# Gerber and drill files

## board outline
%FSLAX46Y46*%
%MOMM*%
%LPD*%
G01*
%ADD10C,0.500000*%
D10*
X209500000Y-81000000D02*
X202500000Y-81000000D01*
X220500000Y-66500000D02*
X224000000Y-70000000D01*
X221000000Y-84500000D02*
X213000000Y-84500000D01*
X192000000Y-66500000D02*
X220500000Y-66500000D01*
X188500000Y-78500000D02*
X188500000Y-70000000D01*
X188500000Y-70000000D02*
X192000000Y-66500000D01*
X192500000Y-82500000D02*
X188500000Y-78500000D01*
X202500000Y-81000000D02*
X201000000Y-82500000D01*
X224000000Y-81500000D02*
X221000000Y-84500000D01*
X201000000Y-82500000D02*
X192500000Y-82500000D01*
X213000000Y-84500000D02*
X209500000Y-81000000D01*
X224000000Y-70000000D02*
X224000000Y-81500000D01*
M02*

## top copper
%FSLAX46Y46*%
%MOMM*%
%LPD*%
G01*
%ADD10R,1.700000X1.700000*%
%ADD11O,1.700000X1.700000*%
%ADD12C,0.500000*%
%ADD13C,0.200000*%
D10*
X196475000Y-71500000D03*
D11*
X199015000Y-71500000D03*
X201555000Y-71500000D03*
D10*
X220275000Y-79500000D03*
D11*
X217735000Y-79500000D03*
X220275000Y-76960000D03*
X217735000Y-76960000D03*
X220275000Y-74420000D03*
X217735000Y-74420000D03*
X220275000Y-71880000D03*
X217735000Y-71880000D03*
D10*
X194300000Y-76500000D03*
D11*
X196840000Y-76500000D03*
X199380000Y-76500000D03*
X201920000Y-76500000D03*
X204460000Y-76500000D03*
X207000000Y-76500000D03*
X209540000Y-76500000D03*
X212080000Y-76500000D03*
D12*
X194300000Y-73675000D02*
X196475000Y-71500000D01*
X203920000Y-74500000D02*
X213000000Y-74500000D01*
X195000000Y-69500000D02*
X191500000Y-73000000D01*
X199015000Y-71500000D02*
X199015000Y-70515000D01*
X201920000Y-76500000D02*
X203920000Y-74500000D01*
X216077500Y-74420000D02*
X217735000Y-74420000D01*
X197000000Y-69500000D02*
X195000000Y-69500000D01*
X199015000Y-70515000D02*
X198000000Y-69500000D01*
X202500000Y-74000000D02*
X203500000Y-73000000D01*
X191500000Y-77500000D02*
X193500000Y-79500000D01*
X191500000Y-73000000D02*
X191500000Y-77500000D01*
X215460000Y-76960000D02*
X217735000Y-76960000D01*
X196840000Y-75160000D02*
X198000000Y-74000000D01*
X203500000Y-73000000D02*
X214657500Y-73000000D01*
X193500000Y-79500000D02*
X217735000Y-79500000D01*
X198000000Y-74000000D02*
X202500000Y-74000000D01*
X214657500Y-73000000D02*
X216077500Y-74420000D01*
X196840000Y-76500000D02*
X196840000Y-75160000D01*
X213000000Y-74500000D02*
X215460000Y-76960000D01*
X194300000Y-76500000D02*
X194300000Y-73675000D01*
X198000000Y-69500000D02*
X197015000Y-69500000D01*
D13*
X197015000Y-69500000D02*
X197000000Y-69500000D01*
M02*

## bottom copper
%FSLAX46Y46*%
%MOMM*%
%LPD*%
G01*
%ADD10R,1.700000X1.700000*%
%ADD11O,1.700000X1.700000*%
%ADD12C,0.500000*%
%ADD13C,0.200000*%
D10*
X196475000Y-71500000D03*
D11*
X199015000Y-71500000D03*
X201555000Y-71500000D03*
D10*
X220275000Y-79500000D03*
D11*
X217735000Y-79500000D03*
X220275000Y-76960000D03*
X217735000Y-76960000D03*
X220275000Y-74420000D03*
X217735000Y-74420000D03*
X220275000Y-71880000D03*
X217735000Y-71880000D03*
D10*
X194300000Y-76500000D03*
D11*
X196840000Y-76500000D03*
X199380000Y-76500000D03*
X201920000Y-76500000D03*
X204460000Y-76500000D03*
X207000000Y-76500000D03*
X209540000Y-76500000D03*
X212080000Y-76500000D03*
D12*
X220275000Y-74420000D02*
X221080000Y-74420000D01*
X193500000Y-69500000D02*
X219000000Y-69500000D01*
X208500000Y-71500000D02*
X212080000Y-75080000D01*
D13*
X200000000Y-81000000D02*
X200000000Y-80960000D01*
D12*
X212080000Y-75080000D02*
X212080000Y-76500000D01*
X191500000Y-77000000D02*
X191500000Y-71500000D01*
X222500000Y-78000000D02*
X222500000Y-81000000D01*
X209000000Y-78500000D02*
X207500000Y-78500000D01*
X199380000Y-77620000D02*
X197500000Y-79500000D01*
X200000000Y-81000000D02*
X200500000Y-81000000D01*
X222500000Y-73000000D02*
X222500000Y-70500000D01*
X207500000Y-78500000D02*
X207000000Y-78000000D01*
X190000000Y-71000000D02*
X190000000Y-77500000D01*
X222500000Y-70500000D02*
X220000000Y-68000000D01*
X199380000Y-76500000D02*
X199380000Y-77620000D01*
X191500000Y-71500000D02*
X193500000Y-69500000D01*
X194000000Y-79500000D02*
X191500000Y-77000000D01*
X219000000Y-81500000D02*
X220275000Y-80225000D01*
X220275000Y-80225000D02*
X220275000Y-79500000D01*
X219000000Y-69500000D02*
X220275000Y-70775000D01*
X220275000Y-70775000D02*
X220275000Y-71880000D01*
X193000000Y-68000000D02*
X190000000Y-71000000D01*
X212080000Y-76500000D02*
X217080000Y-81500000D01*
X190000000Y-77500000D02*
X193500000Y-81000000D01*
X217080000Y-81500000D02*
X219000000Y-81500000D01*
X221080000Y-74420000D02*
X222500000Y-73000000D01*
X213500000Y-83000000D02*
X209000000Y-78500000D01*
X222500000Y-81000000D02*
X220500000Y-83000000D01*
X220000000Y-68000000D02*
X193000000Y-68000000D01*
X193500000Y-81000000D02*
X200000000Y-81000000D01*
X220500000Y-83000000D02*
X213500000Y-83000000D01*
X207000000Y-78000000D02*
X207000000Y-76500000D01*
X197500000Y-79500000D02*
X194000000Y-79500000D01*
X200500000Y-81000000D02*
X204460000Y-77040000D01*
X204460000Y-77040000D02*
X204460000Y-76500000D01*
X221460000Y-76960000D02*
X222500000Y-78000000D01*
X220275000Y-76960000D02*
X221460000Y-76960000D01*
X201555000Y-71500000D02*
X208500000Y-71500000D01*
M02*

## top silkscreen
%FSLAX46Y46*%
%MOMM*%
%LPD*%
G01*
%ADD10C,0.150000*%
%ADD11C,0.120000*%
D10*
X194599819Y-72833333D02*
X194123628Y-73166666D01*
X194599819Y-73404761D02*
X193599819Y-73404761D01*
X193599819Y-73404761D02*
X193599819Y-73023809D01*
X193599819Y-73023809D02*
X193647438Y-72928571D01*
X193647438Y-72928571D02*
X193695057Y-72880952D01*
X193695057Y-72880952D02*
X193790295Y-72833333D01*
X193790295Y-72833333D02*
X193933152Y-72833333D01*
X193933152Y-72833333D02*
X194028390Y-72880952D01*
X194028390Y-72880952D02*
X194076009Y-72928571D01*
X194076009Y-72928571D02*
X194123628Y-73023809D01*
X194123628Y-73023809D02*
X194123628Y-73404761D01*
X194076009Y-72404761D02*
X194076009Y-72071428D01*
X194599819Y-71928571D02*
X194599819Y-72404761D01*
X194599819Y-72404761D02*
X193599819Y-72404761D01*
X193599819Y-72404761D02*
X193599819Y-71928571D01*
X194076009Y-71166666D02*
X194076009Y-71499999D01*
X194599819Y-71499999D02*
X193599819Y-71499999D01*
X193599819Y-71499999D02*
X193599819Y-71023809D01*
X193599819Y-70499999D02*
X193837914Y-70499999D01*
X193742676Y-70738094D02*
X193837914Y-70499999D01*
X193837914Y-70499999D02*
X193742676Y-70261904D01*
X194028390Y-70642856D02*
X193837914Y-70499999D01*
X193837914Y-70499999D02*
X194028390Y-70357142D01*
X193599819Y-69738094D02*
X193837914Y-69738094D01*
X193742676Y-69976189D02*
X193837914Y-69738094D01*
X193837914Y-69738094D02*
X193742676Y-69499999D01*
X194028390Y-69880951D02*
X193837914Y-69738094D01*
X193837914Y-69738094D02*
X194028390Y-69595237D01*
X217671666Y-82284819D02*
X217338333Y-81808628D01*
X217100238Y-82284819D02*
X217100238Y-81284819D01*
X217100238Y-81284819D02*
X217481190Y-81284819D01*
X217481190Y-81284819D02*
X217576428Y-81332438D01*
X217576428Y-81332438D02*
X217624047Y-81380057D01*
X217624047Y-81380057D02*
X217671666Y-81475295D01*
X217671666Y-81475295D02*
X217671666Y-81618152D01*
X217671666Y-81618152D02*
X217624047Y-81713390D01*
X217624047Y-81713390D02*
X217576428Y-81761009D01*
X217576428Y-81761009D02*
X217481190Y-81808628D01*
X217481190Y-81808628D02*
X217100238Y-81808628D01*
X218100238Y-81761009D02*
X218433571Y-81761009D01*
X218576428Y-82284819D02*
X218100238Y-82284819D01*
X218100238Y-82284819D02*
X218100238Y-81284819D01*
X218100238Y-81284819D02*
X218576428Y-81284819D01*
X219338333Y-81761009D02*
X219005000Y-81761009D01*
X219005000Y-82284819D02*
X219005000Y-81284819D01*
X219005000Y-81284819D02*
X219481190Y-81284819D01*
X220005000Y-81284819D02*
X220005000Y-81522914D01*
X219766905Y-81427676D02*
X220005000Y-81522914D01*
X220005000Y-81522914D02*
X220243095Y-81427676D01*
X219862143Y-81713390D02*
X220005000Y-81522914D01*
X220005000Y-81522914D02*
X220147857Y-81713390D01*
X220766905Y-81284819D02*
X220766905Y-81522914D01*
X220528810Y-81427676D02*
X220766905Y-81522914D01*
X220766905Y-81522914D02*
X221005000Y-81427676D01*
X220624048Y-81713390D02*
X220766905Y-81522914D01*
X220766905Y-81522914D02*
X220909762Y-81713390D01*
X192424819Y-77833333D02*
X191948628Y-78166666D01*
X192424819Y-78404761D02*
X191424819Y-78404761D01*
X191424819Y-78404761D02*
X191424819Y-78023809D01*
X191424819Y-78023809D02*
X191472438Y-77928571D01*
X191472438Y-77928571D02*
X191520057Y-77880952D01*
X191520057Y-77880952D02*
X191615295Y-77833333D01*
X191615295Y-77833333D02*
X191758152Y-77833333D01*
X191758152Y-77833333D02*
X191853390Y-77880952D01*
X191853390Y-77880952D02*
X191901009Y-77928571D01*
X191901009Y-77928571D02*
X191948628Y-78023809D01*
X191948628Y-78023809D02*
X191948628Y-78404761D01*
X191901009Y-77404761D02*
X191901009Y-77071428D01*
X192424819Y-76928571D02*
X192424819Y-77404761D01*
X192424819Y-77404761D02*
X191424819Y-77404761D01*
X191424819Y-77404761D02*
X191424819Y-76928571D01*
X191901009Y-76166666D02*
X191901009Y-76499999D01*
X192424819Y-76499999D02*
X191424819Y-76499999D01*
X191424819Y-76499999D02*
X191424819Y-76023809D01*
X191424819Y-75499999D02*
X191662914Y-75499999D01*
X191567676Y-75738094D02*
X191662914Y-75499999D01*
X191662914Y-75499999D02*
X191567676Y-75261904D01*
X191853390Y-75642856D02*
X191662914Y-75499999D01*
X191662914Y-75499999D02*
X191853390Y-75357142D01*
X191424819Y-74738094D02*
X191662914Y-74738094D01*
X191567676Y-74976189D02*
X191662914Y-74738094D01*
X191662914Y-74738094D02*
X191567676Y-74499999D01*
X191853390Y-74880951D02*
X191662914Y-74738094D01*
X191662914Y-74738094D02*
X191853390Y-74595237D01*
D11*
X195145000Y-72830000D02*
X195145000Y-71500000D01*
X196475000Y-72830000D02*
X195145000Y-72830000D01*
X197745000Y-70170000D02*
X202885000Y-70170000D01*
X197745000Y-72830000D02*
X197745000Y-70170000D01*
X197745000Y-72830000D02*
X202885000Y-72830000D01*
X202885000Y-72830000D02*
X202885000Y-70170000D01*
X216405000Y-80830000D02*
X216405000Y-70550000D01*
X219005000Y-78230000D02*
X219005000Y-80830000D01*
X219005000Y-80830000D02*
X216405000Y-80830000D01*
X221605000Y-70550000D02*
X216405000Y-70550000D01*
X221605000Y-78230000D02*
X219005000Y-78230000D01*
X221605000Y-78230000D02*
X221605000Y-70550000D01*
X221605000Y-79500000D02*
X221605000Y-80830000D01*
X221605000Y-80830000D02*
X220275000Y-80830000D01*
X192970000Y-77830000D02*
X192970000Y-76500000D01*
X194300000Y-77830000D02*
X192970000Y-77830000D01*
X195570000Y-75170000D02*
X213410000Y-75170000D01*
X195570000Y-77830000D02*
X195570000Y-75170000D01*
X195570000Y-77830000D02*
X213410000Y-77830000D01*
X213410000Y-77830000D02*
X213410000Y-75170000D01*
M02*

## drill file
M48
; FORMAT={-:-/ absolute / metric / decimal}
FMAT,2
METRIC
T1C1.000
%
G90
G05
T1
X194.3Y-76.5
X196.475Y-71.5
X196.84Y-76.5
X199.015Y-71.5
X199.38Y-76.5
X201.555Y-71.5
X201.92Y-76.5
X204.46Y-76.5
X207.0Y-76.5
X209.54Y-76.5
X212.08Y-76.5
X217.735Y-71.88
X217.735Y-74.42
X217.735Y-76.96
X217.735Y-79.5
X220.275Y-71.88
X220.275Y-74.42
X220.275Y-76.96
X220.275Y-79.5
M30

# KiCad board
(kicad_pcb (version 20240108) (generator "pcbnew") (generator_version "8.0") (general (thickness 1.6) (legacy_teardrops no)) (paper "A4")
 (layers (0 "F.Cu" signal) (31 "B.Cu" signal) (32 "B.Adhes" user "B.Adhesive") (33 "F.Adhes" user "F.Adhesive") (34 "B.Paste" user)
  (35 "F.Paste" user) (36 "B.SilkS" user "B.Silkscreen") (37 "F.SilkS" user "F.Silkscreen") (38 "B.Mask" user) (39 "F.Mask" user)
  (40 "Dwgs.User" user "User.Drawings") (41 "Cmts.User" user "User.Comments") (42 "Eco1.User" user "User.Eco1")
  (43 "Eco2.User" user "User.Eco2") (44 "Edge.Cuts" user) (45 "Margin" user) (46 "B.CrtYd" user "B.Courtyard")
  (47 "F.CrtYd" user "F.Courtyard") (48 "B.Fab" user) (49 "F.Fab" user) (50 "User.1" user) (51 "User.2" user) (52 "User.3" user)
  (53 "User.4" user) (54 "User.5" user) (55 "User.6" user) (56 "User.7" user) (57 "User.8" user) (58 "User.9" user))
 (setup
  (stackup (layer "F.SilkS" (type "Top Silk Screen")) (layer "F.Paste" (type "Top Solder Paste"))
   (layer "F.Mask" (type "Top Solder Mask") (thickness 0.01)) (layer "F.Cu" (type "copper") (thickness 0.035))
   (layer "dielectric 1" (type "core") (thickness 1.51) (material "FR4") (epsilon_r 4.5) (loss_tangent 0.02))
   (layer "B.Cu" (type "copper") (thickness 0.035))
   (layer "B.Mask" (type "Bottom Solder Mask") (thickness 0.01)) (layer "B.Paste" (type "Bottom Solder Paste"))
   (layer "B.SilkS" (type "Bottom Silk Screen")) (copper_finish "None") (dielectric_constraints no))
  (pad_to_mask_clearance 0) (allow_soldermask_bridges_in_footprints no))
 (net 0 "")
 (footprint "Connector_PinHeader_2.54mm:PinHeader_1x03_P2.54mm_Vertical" (layer "F.Cu") (at 196.475 71.5 90)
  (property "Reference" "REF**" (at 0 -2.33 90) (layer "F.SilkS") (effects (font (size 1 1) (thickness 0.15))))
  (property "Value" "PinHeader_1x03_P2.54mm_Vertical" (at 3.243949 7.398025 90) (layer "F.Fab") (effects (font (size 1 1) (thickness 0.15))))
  (fp_line (start -1.33 -1.33) (end 0 -1.33) (stroke (width 0.12) (type solid)) (layer "F.SilkS"))
  (fp_line (start -1.33 0) (end -1.33 -1.33) (stroke (width 0.12) (type solid)) (layer "F.SilkS"))
  (fp_line (start 1.33 1.27) (end 1.33 6.41) (stroke (width 0.12) (type solid)) (layer "F.SilkS"))
  (fp_line (start -1.33 1.27) (end 1.33 1.27) (stroke (width 0.12) (type solid)) (layer "F.SilkS"))
  (fp_line (start -1.33 1.27) (end -1.33 6.41) (stroke (width 0.12) (type solid)) (layer "F.SilkS"))
  (fp_line (start -1.33 6.41) (end 1.33 6.41) (stroke (width 0.12) (type solid)) (layer "F.SilkS"))
  (pad "1" thru_hole rect (at 0 0 90) (size 1.7 1.7) (drill 1) (layers "*.Cu" "*.Mask") (remove_unused_layers no))
  (pad "2" thru_hole oval (at 0 2.54 90) (size 1.7 1.7) (drill 1) (layers "*.Cu" "*.Mask") (remove_unused_layers no))
  (pad "3" thru_hole oval (at 0 5.08 90) (size 1.7 1.7) (drill 1) (layers "*.Cu" "*.Mask") (remove_unused_layers no)))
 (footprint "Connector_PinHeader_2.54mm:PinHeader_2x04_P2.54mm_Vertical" (layer "F.Cu") (at 220.275 79.5 180)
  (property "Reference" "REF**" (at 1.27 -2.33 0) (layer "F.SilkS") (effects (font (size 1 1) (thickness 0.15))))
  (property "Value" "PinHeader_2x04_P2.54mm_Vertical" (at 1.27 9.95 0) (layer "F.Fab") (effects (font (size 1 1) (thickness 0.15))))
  (fp_line (start 3.87 -1.33) (end 3.87 8.95) (stroke (width 0.12) (type solid)) (layer "F.SilkS"))
  (fp_line (start 1.27 1.27) (end 1.27 -1.33) (stroke (width 0.12) (type solid)) (layer "F.SilkS"))
  (fp_line (start 1.27 -1.33) (end 3.87 -1.33) (stroke (width 0.12) (type solid)) (layer "F.SilkS"))
  (fp_line (start -1.33 8.95) (end 3.87 8.95) (stroke (width 0.12) (type solid)) (layer "F.SilkS"))
  (fp_line (start -1.33 1.27) (end 1.27 1.27) (stroke (width 0.12) (type solid)) (layer "F.SilkS"))
  (fp_line (start -1.33 1.27) (end -1.33 8.95) (stroke (width 0.12) (type solid)) (layer "F.SilkS"))
  (fp_line (start -1.33 0) (end -1.33 -1.33) (stroke (width 0.12) (type solid)) (layer "F.SilkS"))
  (fp_line (start -1.33 -1.33) (end 0 -1.33) (stroke (width 0.12) (type solid)) (layer "F.SilkS"))
  (pad "1" thru_hole rect (at 0 0 180) (size 1.7 1.7) (drill 1) (layers "*.Cu" "*.Mask") (remove_unused_layers no))
  (pad "2" thru_hole oval (at 2.54 0 180) (size 1.7 1.7) (drill 1) (layers "*.Cu" "*.Mask") (remove_unused_layers no))
  (pad "3" thru_hole oval (at 0 2.54 180) (size 1.7 1.7) (drill 1) (layers "*.Cu" "*.Mask") (remove_unused_layers no))
  (pad "4" thru_hole oval (at 2.54 2.54 180) (size 1.7 1.7) (drill 1) (layers "*.Cu" "*.Mask") (remove_unused_layers no))
  (pad "5" thru_hole oval (at 0 5.08 180) (size 1.7 1.7) (drill 1) (layers "*.Cu" "*.Mask") (remove_unused_layers no))
  (pad "6" thru_hole oval (at 2.54 5.08 180) (size 1.7 1.7) (drill 1) (layers "*.Cu" "*.Mask") (remove_unused_layers no))
  (pad "7" thru_hole oval (at 0 7.62 180) (size 1.7 1.7) (drill 1) (layers "*.Cu" "*.Mask") (remove_unused_layers no))
  (pad "8" thru_hole oval (at 2.54 7.62 180) (size 1.7 1.7) (drill 1) (layers "*.Cu" "*.Mask") (remove_unused_layers no)))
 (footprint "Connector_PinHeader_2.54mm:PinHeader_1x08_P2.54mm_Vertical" (layer "F.Cu") (at 194.3 76.5 90)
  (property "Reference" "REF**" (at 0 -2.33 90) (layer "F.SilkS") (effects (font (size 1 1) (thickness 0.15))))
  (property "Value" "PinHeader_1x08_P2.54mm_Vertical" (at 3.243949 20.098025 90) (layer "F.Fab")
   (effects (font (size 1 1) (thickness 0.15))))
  (fp_line (start -1.33 -1.33) (end 0 -1.33) (stroke (width 0.12) (type solid)) (layer "F.SilkS"))
  (fp_line (start -1.33 0) (end -1.33 -1.33) (stroke (width 0.12) (type solid)) (layer "F.SilkS"))
  (fp_line (start 1.33 1.27) (end 1.33 19.11) (stroke (width 0.12) (type solid)) (layer "F.SilkS"))
  (fp_line (start -1.33 1.27) (end 1.33 1.27) (stroke (width 0.12) (type solid)) (layer "F.SilkS"))
  (fp_line (start -1.33 1.27) (end -1.33 19.11) (stroke (width 0.12) (type solid)) (layer "F.SilkS"))
  (fp_line (start -1.33 19.11) (end 1.33 19.11) (stroke (width 0.12) (type solid)) (layer "F.SilkS"))
  (pad "1" thru_hole rect (at 0 0 90) (size 1.7 1.7) (drill 1) (layers "*.Cu" "*.Mask") (remove_unused_layers no))
  (pad "2" thru_hole oval (at 0 2.54 90) (size 1.7 1.7) (drill 1) (layers "*.Cu" "*.Mask") (remove_unused_layers no))
  (pad "3" thru_hole oval (at 0 5.08 90) (size 1.7 1.7) (drill 1) (layers "*.Cu" "*.Mask") (remove_unused_layers no))
  (pad "4" thru_hole oval (at 0 7.62 90) (size 1.7 1.7) (drill 1) (layers "*.Cu" "*.Mask") (remove_unused_layers no))
  (pad "5" thru_hole oval (at 0 10.16 90) (size 1.7 1.7) (drill 1) (layers "*.Cu" "*.Mask") (remove_unused_layers no))
  (pad "6" thru_hole oval (at 0 12.7 90) (size 1.7 1.7) (drill 1) (layers "*.Cu" "*.Mask") (remove_unused_layers no))
  (pad "7" thru_hole oval (at 0 15.24 90) (size 1.7 1.7) (drill 1) (layers "*.Cu" "*.Mask") (remove_unused_layers no))
  (pad "8" thru_hole oval (at 0 17.78 90) (size 1.7 1.7) (drill 1) (layers "*.Cu" "*.Mask") (remove_unused_layers no)))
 (gr_line (start 209.5 81) (end 202.5 81) (stroke (width 0.5) (type default)) (layer "Edge.Cuts"))
 (gr_line (start 220.5 66.5) (end 224 70) (stroke (width 0.5) (type default)) (layer "Edge.Cuts"))
 (gr_line (start 221 84.5) (end 213 84.5) (stroke (width 0.5) (type default)) (layer "Edge.Cuts"))
 (gr_line (start 192 66.5) (end 220.5 66.5) (stroke (width 0.5) (type default)) (layer "Edge.Cuts"))
 (gr_line (start 188.5 78.5) (end 188.5 70) (stroke (width 0.5) (type default)) (layer "Edge.Cuts"))
 (gr_line (start 188.5 70) (end 192 66.5) (stroke (width 0.5) (type default)) (layer "Edge.Cuts"))
 (gr_line (start 192.5 82.5) (end 188.5 78.5) (stroke (width 0.5) (type default)) (layer "Edge.Cuts"))
 (gr_line (start 202.5 81) (end 201 82.5) (stroke (width 0.5) (type default)) (layer "Edge.Cuts"))
 (gr_line (start 224 81.5) (end 221 84.5) (stroke (width 0.5) (type default)) (layer "Edge.Cuts"))
 (gr_line (start 201 82.5) (end 192.5 82.5) (stroke (width 0.5) (type default)) (layer "Edge.Cuts"))
 (gr_line (start 213 84.5) (end 209.5 81) (stroke (width 0.5) (type default)) (layer "Edge.Cuts"))
 (gr_line (start 224 70) (end 224 81.5) (stroke (width 0.5) (type default)) (layer "Edge.Cuts"))
 (segment (start 194.3 73.675) (end 196.475 71.5) (width 0.5) (layer "F.Cu") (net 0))
 (segment (start 203.92 74.5) (end 213 74.5) (width 0.5) (layer "F.Cu") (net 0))
 (segment (start 195 69.5) (end 191.5 73) (width 0.5) (layer "F.Cu") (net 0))
 (segment (start 199.015 71.5) (end 199.015 70.515) (width 0.5) (layer "F.Cu") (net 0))
 (segment (start 201.92 76.5) (end 203.92 74.5) (width 0.5) (layer "F.Cu") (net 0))
 (segment (start 216.0775 74.42) (end 217.735 74.42) (width 0.5) (layer "F.Cu") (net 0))
 (segment (start 197 69.5) (end 195 69.5) (width 0.5) (layer "F.Cu") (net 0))
 (segment (start 199.015 70.515) (end 198 69.5) (width 0.5) (layer "F.Cu") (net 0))
 (segment (start 202.5 74) (end 203.5 73) (width 0.5) (layer "F.Cu") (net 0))
 (segment (start 191.5 77.5) (end 193.5 79.5) (width 0.5) (layer "F.Cu") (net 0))
 (segment (start 191.5 73) (end 191.5 77.5) (width 0.5) (layer "F.Cu") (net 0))
 (segment (start 215.46 76.96) (end 217.735 76.96) (width 0.5) (layer "F.Cu") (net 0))
 (segment (start 196.84 75.16) (end 198 74) (width 0.5) (layer "F.Cu") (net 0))
 (segment (start 203.5 73) (end 214.6575 73) (width 0.5) (layer "F.Cu") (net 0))
 (segment (start 193.5 79.5) (end 217.735 79.5) (width 0.5) (layer "F.Cu") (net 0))
 (segment (start 198 74) (end 202.5 74) (width 0.5) (layer "F.Cu") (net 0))
 (segment (start 214.6575 73) (end 216.0775 74.42) (width 0.5) (layer "F.Cu") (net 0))
 (segment (start 196.84 76.5) (end 196.84 75.16) (width 0.5) (layer "F.Cu") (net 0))
 (segment (start 213 74.5) (end 215.46 76.96) (width 0.5) (layer "F.Cu") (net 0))
 (segment (start 194.3 76.5) (end 194.3 73.675) (width 0.5) (layer "F.Cu") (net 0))
 (segment (start 198 69.5) (end 197.015 69.5) (width 0.5) (layer "F.Cu") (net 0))
 (segment (start 197.015 69.5) (end 197 69.5) (width 0.2) (layer "F.Cu") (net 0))
 (segment (start 220.275 74.42) (end 221.08 74.42) (width 0.5) (layer "B.Cu") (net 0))
 (segment (start 193.5 69.5) (end 219 69.5) (width 0.5) (layer "B.Cu") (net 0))
 (segment (start 208.5 71.5) (end 212.08 75.08) (width 0.5) (layer "B.Cu") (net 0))
 (segment (start 200 81) (end 200 80.96) (width 0.2) (layer "B.Cu") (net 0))
 (segment (start 212.08 75.08) (end 212.08 76.5) (width 0.5) (layer "B.Cu") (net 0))
 (segment (start 191.5 77) (end 191.5 71.5) (width 0.5) (layer "B.Cu") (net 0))
 (segment (start 222.5 78) (end 222.5 81) (width 0.5) (layer "B.Cu") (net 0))
 (segment (start 209 78.5) (end 207.5 78.5) (width 0.5) (layer "B.Cu") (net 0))
 (segment (start 199.38 77.62) (end 197.5 79.5) (width 0.5) (layer "B.Cu") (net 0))
 (segment (start 200 81) (end 200.5 81) (width 0.5) (layer "B.Cu") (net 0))
 (segment (start 222.5 73) (end 222.5 70.5) (width 0.5) (layer "B.Cu") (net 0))
 (segment (start 207.5 78.5) (end 207 78) (width 0.5) (layer "B.Cu") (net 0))
 (segment (start 190 71) (end 190 77.5) (width 0.5) (layer "B.Cu") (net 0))
 (segment (start 222.5 70.5) (end 220 68) (width 0.5) (layer "B.Cu") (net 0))
 (segment (start 199.38 76.5) (end 199.38 77.62) (width 0.5) (layer "B.Cu") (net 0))
 (segment (start 191.5 71.5) (end 193.5 69.5) (width 0.5) (layer "B.Cu") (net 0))
 (segment (start 194 79.5) (end 191.5 77) (width 0.5) (layer "B.Cu") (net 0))
 (segment (start 219 81.5) (end 220.275 80.225) (width 0.5) (layer "B.Cu") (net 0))
 (segment (start 220.275 80.225) (end 220.275 79.5) (width 0.5) (layer "B.Cu") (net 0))
 (segment (start 219 69.5) (end 220.275 70.775) (width 0.5) (layer "B.Cu") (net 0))
 (segment (start 220.275 70.775) (end 220.275 71.88) (width 0.5) (layer "B.Cu") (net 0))
 (segment (start 193 68) (end 190 71) (width 0.5) (layer "B.Cu") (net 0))
 (segment (start 212.08 76.5) (end 217.08 81.5) (width 0.5) (layer "B.Cu") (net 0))
 (segment (start 190 77.5) (end 193.5 81) (width 0.5) (layer "B.Cu") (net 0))
 (segment (start 217.08 81.5) (end 219 81.5) (width 0.5) (layer "B.Cu") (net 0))
 (segment (start 221.08 74.42) (end 222.5 73) (width 0.5) (layer "B.Cu") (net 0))
 (segment (start 213.5 83) (end 209 78.5) (width 0.5) (layer "B.Cu") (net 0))
 (segment (start 222.5 81) (end 220.5 83) (width 0.5) (layer "B.Cu") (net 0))
 (segment (start 220 68) (end 193 68) (width 0.5) (layer "B.Cu") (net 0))
 (segment (start 193.5 81) (end 200 81) (width 0.5) (layer "B.Cu") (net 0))
 (segment (start 220.5 83) (end 213.5 83) (width 0.5) (layer "B.Cu") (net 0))
 (segment (start 207 78) (end 207 76.5) (width 0.5) (layer "B.Cu") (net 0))
 (segment (start 197.5 79.5) (end 194 79.5) (width 0.5) (layer "B.Cu") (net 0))
 (segment (start 200.5 81) (end 204.46 77.04) (width 0.5) (layer "B.Cu") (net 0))
 (segment (start 204.46 77.04) (end 204.46 76.5) (width 0.5) (layer "B.Cu") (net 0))
 (segment (start 221.46 76.96) (end 222.5 78) (width 0.5) (layer "B.Cu") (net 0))
 (segment (start 220.275 76.96) (end 221.46 76.96) (width 0.5) (layer "B.Cu") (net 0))
 (segment (start 201.555 71.5) (end 208.5 71.5) (width 0.5) (layer "B.Cu") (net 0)))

